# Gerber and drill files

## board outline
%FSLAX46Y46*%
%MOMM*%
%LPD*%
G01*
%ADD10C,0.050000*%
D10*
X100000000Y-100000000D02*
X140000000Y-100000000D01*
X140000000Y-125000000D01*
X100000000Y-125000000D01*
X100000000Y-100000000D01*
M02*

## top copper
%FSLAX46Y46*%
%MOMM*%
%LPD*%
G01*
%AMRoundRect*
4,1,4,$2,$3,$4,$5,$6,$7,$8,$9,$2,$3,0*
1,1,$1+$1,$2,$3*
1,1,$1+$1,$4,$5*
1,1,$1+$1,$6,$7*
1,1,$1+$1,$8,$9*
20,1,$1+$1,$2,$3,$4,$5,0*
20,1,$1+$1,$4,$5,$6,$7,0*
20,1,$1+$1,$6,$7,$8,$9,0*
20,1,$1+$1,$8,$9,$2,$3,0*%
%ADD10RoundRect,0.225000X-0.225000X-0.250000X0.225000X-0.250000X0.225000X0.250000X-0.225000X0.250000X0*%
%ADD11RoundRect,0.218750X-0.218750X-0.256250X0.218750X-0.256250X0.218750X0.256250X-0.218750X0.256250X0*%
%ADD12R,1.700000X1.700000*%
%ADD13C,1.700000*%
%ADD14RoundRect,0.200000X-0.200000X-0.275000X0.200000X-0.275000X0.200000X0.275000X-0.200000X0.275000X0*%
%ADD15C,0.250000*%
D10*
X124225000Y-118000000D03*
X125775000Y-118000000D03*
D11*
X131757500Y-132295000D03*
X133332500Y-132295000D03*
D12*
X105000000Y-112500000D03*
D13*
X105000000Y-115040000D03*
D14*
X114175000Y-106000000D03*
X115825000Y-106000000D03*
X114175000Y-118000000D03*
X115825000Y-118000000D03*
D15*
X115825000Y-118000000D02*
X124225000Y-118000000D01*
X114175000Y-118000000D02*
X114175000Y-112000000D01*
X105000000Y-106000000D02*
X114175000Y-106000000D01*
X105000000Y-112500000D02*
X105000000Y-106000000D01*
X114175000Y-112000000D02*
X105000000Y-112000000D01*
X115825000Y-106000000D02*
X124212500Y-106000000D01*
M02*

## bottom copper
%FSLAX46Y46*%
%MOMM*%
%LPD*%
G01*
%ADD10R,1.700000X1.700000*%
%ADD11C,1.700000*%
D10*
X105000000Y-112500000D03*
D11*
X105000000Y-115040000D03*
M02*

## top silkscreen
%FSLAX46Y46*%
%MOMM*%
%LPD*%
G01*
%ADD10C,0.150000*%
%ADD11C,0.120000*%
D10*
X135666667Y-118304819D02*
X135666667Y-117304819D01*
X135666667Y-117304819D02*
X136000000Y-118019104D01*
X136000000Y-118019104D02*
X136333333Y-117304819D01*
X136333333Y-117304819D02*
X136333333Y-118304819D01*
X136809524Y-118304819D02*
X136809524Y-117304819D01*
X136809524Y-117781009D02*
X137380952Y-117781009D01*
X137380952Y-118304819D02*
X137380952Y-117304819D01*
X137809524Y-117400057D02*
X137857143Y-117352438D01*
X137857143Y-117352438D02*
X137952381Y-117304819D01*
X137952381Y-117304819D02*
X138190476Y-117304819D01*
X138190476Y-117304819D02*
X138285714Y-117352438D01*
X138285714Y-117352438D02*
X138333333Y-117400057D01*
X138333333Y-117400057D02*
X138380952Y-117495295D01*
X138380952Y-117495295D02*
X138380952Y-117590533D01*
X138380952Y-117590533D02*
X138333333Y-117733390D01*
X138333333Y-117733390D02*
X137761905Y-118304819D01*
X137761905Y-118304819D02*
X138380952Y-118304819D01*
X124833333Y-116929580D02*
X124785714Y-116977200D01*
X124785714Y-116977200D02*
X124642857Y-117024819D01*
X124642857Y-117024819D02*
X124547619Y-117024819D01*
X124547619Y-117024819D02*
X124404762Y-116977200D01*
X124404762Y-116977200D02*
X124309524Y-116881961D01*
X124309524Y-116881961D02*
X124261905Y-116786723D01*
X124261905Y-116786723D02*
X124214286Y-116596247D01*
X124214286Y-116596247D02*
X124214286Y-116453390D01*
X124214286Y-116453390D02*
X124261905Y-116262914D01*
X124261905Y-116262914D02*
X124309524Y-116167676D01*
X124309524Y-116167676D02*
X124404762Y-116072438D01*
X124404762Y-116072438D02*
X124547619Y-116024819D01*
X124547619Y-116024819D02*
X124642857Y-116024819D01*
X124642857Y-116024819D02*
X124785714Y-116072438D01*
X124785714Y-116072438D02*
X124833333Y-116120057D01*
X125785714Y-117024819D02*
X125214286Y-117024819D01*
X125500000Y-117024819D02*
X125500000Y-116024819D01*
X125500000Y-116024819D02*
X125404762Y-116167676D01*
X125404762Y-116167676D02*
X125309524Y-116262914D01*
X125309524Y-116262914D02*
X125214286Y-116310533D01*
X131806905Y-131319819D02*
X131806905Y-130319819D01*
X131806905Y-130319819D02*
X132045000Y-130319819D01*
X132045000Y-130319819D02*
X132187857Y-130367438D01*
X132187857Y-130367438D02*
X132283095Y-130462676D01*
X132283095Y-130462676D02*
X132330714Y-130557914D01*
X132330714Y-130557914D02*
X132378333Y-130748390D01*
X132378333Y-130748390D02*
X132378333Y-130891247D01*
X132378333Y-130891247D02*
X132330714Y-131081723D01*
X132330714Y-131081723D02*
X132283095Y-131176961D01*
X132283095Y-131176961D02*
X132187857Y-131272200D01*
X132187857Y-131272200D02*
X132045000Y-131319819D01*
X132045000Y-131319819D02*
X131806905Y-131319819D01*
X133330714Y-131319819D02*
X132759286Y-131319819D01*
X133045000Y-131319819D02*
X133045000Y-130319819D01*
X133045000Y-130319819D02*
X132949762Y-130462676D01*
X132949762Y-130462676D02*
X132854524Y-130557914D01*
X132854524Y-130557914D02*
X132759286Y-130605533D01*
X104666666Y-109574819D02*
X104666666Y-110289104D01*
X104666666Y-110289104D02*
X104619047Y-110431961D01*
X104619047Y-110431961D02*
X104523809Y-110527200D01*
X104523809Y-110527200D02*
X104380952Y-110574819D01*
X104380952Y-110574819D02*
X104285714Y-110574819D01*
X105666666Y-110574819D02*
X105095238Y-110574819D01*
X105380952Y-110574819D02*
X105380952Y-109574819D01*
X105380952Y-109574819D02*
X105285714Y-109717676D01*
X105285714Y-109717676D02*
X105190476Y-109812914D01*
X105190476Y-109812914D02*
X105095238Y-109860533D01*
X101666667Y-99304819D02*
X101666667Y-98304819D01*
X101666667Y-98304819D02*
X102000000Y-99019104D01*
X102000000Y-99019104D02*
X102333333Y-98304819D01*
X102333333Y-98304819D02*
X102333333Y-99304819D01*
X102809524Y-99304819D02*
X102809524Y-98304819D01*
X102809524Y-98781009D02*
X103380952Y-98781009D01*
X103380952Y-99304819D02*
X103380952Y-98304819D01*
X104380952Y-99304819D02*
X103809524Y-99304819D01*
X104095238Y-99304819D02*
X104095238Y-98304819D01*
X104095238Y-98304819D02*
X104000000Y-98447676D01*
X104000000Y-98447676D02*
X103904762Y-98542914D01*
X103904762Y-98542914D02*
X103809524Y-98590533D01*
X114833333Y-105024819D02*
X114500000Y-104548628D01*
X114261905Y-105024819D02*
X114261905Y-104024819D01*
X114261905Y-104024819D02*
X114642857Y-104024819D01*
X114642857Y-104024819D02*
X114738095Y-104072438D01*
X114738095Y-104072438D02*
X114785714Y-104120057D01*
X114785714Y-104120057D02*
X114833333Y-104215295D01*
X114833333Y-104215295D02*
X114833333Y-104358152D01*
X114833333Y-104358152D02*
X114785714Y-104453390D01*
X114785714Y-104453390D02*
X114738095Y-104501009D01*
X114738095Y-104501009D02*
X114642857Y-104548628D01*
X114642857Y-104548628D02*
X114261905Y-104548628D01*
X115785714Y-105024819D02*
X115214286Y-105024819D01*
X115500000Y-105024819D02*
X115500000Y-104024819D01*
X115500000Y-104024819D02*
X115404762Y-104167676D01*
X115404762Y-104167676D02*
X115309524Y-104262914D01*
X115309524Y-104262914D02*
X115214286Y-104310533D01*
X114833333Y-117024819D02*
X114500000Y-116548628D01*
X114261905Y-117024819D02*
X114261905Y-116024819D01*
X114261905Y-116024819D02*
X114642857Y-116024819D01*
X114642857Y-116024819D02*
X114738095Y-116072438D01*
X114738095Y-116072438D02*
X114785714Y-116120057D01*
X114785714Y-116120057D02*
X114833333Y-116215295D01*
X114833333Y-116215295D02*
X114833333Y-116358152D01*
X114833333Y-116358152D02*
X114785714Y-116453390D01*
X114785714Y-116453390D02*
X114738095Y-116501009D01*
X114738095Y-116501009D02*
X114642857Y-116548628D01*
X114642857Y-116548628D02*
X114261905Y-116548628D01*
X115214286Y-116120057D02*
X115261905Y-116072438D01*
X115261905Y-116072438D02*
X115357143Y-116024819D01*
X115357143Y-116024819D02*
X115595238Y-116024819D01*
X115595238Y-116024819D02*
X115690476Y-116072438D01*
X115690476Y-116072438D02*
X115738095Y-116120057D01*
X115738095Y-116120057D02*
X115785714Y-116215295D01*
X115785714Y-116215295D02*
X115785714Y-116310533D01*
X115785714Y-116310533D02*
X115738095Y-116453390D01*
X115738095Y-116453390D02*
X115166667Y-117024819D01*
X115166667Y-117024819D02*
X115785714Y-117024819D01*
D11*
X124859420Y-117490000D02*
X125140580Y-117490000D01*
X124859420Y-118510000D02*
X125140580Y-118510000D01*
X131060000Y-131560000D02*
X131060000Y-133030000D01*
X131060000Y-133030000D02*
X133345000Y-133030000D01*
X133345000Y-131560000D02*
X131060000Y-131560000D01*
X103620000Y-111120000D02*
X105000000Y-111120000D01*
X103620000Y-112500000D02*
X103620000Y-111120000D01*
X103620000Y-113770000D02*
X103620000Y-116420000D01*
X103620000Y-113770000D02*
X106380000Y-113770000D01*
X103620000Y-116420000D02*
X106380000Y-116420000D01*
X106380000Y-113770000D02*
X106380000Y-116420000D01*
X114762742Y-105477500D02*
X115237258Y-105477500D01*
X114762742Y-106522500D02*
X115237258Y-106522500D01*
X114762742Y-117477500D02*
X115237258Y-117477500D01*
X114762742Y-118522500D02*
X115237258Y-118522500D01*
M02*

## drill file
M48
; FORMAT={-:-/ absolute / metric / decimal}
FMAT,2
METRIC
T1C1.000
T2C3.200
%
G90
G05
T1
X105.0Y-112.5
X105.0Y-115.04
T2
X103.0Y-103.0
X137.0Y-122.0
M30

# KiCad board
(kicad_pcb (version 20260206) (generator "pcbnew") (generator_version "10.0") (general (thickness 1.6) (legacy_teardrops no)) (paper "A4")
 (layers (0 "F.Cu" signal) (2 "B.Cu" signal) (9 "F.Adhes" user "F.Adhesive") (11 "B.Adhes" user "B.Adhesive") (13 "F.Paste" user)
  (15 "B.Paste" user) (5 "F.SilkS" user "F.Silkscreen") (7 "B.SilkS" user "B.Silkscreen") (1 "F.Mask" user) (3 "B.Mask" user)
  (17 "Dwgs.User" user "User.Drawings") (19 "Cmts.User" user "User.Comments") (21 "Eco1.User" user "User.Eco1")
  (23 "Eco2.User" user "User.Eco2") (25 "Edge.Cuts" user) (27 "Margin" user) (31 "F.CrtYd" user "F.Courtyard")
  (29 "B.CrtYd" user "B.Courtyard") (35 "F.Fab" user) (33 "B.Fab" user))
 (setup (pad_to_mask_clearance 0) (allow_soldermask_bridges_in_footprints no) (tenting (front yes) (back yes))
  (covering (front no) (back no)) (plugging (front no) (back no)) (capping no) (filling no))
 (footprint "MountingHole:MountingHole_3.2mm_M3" (layer "F.Cu") (at 137 122)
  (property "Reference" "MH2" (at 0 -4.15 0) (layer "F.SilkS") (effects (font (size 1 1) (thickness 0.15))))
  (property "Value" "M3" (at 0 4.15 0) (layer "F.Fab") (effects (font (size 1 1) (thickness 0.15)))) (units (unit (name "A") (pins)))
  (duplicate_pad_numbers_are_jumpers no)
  (pad "" np_thru_hole circle (at 0 0) (size 3.2 3.2) (drill 3.2) (layers "*.Cu" "*.Mask")))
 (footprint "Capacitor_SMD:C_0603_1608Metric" (layer "F.Cu") (at 125 118)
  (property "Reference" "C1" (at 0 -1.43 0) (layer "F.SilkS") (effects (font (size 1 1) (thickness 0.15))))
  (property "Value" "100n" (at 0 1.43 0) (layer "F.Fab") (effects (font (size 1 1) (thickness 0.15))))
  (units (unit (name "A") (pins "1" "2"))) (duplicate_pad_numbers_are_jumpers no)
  (fp_line (start -0.14058 -0.51) (end 0.14058 -0.51) (stroke (width 0.12) (type solid)) (layer "F.SilkS"))
  (fp_line (start -0.14058 0.51) (end 0.14058 0.51) (stroke (width 0.12) (type solid)) (layer "F.SilkS"))
  (pad "1" smd roundrect (at -0.775 0) (size 0.9 0.95) (layers "F.Cu" "F.Mask" "F.Paste") (roundrect_rratio 0.25) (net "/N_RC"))
  (pad "2" smd roundrect (at 0.775 0) (size 0.9 0.95) (layers "F.Cu" "F.Mask" "F.Paste") (roundrect_rratio 0.25) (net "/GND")))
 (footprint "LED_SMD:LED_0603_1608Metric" (layer "F.Cu") (at 132.545 132.295)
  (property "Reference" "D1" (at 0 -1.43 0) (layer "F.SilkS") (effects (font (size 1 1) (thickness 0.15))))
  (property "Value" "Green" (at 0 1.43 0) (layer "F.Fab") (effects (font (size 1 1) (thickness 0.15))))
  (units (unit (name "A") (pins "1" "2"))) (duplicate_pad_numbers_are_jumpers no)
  (fp_line (start -1.485 -0.735) (end -1.485 0.735) (stroke (width 0.12) (type solid)) (layer "F.SilkS"))
  (fp_line (start -1.485 0.735) (end 0.8 0.735) (stroke (width 0.12) (type solid)) (layer "F.SilkS"))
  (fp_line (start 0.8 -0.735) (end -1.485 -0.735) (stroke (width 0.12) (type solid)) (layer "F.SilkS"))
  (pad "1" smd roundrect (at -0.7875 0) (size 0.875 0.95) (layers "F.Cu" "F.Mask" "F.Paste") (roundrect_rratio 0.25) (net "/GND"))
  (pad "2" smd roundrect (at 0.7875 0) (size 0.875 0.95) (layers "F.Cu" "F.Mask" "F.Paste") (roundrect_rratio 0.25) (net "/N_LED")))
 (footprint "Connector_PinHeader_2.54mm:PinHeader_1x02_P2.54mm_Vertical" (layer "F.Cu") (at 105 112.5)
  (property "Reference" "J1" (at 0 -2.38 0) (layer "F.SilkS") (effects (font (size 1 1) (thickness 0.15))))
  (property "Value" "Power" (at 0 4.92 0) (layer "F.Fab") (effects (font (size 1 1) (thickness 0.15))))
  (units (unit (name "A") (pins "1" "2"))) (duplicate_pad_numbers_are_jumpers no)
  (fp_line (start -1.38 -1.38) (end 0 -1.38) (stroke (width 0.12) (type solid)) (layer "F.SilkS"))
  (fp_line (start -1.38 0) (end -1.38 -1.38) (stroke (width 0.12) (type solid)) (layer "F.SilkS"))
  (fp_line (start -1.38 1.27) (end -1.38 3.92) (stroke (width 0.12) (type solid)) (layer "F.SilkS"))
  (fp_line (start -1.38 1.27) (end 1.38 1.27) (stroke (width 0.12) (type solid)) (layer "F.SilkS"))
  (fp_line (start -1.38 3.92) (end 1.38 3.92) (stroke (width 0.12) (type solid)) (layer "F.SilkS"))
  (fp_line (start 1.38 1.27) (end 1.38 3.92) (stroke (width 0.12) (type solid)) (layer "F.SilkS"))
  (pad "1" thru_hole rect (at 0 0) (size 1.7 1.7) (drill 1) (layers "*.Cu" "*.Mask") (remove_unused_layers no) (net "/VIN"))
  (pad "2" thru_hole circle (at 0 2.54) (size 1.7 1.7) (drill 1) (layers "*.Cu" "*.Mask") (remove_unused_layers no) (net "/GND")))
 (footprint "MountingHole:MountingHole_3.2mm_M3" (layer "F.Cu") (at 103 103)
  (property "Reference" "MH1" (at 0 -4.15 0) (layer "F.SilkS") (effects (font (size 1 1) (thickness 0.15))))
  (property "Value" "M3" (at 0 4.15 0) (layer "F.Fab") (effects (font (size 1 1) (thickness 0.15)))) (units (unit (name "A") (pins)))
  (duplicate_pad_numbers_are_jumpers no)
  (pad "" np_thru_hole circle (at 0 0) (size 3.2 3.2) (drill 3.2) (layers "*.Cu" "*.Mask")))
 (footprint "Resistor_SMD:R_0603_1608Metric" (layer "F.Cu") (at 115 106)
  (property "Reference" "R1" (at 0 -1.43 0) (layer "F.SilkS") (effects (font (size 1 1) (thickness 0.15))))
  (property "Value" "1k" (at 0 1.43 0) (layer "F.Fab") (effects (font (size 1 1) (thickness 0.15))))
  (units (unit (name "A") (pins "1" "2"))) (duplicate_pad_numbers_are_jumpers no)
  (fp_line (start -0.237258 -0.5225) (end 0.237258 -0.5225) (stroke (width 0.12) (type solid)) (layer "F.SilkS"))
  (fp_line (start -0.237258 0.5225) (end 0.237258 0.5225) (stroke (width 0.12) (type solid)) (layer "F.SilkS"))
  (pad "1" smd roundrect (at -0.825 0) (size 0.8 0.95) (layers "F.Cu" "F.Mask" "F.Paste") (roundrect_rratio 0.25) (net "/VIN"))
  (pad "2" smd roundrect (at 0.825 0) (size 0.8 0.95) (layers "F.Cu" "F.Mask" "F.Paste") (roundrect_rratio 0.25) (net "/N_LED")))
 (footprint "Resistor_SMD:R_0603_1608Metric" (layer "F.Cu") (at 115 118)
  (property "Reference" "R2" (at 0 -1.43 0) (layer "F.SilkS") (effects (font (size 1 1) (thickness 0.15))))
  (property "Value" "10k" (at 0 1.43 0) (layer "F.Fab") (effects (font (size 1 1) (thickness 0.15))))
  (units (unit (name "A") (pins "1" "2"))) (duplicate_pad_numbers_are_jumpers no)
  (fp_line (start -0.237258 -0.5225) (end 0.237258 -0.5225) (stroke (width 0.12) (type solid)) (layer "F.SilkS"))
  (fp_line (start -0.237258 0.5225) (end 0.237258 0.5225) (stroke (width 0.12) (type solid)) (layer "F.SilkS"))
  (pad "1" smd roundrect (at -0.825 0) (size 0.8 0.95) (layers "F.Cu" "F.Mask" "F.Paste") (roundrect_rratio 0.25) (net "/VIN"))
  (pad "2" smd roundrect (at 0.825 0) (size 0.8 0.95) (layers "F.Cu" "F.Mask" "F.Paste") (roundrect_rratio 0.25) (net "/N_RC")))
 (gr_rect (start 100 100) (end 140 125) (stroke (width 0.05) (type default)) (fill no) (layer "Edge.Cuts"))
 (segment (start 115.825 118) (end 124.225 118) (width 0.25) (layer "F.Cu") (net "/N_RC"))
 (segment (start 114.175 118) (end 114.175 112) (width 0.25) (layer "F.Cu") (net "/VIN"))
 (segment (start 105 106) (end 114.175 106) (width 0.25) (layer "F.Cu") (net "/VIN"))
 (segment (start 105 112.5) (end 105 106) (width 0.25) (layer "F.Cu") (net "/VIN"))
 (segment (start 114.175 112) (end 105 112) (width 0.25) (layer "F.Cu") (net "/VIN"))
 (segment (start 115.825 106) (end 124.2125 106) (width 0.25) (layer "F.Cu") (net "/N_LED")))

